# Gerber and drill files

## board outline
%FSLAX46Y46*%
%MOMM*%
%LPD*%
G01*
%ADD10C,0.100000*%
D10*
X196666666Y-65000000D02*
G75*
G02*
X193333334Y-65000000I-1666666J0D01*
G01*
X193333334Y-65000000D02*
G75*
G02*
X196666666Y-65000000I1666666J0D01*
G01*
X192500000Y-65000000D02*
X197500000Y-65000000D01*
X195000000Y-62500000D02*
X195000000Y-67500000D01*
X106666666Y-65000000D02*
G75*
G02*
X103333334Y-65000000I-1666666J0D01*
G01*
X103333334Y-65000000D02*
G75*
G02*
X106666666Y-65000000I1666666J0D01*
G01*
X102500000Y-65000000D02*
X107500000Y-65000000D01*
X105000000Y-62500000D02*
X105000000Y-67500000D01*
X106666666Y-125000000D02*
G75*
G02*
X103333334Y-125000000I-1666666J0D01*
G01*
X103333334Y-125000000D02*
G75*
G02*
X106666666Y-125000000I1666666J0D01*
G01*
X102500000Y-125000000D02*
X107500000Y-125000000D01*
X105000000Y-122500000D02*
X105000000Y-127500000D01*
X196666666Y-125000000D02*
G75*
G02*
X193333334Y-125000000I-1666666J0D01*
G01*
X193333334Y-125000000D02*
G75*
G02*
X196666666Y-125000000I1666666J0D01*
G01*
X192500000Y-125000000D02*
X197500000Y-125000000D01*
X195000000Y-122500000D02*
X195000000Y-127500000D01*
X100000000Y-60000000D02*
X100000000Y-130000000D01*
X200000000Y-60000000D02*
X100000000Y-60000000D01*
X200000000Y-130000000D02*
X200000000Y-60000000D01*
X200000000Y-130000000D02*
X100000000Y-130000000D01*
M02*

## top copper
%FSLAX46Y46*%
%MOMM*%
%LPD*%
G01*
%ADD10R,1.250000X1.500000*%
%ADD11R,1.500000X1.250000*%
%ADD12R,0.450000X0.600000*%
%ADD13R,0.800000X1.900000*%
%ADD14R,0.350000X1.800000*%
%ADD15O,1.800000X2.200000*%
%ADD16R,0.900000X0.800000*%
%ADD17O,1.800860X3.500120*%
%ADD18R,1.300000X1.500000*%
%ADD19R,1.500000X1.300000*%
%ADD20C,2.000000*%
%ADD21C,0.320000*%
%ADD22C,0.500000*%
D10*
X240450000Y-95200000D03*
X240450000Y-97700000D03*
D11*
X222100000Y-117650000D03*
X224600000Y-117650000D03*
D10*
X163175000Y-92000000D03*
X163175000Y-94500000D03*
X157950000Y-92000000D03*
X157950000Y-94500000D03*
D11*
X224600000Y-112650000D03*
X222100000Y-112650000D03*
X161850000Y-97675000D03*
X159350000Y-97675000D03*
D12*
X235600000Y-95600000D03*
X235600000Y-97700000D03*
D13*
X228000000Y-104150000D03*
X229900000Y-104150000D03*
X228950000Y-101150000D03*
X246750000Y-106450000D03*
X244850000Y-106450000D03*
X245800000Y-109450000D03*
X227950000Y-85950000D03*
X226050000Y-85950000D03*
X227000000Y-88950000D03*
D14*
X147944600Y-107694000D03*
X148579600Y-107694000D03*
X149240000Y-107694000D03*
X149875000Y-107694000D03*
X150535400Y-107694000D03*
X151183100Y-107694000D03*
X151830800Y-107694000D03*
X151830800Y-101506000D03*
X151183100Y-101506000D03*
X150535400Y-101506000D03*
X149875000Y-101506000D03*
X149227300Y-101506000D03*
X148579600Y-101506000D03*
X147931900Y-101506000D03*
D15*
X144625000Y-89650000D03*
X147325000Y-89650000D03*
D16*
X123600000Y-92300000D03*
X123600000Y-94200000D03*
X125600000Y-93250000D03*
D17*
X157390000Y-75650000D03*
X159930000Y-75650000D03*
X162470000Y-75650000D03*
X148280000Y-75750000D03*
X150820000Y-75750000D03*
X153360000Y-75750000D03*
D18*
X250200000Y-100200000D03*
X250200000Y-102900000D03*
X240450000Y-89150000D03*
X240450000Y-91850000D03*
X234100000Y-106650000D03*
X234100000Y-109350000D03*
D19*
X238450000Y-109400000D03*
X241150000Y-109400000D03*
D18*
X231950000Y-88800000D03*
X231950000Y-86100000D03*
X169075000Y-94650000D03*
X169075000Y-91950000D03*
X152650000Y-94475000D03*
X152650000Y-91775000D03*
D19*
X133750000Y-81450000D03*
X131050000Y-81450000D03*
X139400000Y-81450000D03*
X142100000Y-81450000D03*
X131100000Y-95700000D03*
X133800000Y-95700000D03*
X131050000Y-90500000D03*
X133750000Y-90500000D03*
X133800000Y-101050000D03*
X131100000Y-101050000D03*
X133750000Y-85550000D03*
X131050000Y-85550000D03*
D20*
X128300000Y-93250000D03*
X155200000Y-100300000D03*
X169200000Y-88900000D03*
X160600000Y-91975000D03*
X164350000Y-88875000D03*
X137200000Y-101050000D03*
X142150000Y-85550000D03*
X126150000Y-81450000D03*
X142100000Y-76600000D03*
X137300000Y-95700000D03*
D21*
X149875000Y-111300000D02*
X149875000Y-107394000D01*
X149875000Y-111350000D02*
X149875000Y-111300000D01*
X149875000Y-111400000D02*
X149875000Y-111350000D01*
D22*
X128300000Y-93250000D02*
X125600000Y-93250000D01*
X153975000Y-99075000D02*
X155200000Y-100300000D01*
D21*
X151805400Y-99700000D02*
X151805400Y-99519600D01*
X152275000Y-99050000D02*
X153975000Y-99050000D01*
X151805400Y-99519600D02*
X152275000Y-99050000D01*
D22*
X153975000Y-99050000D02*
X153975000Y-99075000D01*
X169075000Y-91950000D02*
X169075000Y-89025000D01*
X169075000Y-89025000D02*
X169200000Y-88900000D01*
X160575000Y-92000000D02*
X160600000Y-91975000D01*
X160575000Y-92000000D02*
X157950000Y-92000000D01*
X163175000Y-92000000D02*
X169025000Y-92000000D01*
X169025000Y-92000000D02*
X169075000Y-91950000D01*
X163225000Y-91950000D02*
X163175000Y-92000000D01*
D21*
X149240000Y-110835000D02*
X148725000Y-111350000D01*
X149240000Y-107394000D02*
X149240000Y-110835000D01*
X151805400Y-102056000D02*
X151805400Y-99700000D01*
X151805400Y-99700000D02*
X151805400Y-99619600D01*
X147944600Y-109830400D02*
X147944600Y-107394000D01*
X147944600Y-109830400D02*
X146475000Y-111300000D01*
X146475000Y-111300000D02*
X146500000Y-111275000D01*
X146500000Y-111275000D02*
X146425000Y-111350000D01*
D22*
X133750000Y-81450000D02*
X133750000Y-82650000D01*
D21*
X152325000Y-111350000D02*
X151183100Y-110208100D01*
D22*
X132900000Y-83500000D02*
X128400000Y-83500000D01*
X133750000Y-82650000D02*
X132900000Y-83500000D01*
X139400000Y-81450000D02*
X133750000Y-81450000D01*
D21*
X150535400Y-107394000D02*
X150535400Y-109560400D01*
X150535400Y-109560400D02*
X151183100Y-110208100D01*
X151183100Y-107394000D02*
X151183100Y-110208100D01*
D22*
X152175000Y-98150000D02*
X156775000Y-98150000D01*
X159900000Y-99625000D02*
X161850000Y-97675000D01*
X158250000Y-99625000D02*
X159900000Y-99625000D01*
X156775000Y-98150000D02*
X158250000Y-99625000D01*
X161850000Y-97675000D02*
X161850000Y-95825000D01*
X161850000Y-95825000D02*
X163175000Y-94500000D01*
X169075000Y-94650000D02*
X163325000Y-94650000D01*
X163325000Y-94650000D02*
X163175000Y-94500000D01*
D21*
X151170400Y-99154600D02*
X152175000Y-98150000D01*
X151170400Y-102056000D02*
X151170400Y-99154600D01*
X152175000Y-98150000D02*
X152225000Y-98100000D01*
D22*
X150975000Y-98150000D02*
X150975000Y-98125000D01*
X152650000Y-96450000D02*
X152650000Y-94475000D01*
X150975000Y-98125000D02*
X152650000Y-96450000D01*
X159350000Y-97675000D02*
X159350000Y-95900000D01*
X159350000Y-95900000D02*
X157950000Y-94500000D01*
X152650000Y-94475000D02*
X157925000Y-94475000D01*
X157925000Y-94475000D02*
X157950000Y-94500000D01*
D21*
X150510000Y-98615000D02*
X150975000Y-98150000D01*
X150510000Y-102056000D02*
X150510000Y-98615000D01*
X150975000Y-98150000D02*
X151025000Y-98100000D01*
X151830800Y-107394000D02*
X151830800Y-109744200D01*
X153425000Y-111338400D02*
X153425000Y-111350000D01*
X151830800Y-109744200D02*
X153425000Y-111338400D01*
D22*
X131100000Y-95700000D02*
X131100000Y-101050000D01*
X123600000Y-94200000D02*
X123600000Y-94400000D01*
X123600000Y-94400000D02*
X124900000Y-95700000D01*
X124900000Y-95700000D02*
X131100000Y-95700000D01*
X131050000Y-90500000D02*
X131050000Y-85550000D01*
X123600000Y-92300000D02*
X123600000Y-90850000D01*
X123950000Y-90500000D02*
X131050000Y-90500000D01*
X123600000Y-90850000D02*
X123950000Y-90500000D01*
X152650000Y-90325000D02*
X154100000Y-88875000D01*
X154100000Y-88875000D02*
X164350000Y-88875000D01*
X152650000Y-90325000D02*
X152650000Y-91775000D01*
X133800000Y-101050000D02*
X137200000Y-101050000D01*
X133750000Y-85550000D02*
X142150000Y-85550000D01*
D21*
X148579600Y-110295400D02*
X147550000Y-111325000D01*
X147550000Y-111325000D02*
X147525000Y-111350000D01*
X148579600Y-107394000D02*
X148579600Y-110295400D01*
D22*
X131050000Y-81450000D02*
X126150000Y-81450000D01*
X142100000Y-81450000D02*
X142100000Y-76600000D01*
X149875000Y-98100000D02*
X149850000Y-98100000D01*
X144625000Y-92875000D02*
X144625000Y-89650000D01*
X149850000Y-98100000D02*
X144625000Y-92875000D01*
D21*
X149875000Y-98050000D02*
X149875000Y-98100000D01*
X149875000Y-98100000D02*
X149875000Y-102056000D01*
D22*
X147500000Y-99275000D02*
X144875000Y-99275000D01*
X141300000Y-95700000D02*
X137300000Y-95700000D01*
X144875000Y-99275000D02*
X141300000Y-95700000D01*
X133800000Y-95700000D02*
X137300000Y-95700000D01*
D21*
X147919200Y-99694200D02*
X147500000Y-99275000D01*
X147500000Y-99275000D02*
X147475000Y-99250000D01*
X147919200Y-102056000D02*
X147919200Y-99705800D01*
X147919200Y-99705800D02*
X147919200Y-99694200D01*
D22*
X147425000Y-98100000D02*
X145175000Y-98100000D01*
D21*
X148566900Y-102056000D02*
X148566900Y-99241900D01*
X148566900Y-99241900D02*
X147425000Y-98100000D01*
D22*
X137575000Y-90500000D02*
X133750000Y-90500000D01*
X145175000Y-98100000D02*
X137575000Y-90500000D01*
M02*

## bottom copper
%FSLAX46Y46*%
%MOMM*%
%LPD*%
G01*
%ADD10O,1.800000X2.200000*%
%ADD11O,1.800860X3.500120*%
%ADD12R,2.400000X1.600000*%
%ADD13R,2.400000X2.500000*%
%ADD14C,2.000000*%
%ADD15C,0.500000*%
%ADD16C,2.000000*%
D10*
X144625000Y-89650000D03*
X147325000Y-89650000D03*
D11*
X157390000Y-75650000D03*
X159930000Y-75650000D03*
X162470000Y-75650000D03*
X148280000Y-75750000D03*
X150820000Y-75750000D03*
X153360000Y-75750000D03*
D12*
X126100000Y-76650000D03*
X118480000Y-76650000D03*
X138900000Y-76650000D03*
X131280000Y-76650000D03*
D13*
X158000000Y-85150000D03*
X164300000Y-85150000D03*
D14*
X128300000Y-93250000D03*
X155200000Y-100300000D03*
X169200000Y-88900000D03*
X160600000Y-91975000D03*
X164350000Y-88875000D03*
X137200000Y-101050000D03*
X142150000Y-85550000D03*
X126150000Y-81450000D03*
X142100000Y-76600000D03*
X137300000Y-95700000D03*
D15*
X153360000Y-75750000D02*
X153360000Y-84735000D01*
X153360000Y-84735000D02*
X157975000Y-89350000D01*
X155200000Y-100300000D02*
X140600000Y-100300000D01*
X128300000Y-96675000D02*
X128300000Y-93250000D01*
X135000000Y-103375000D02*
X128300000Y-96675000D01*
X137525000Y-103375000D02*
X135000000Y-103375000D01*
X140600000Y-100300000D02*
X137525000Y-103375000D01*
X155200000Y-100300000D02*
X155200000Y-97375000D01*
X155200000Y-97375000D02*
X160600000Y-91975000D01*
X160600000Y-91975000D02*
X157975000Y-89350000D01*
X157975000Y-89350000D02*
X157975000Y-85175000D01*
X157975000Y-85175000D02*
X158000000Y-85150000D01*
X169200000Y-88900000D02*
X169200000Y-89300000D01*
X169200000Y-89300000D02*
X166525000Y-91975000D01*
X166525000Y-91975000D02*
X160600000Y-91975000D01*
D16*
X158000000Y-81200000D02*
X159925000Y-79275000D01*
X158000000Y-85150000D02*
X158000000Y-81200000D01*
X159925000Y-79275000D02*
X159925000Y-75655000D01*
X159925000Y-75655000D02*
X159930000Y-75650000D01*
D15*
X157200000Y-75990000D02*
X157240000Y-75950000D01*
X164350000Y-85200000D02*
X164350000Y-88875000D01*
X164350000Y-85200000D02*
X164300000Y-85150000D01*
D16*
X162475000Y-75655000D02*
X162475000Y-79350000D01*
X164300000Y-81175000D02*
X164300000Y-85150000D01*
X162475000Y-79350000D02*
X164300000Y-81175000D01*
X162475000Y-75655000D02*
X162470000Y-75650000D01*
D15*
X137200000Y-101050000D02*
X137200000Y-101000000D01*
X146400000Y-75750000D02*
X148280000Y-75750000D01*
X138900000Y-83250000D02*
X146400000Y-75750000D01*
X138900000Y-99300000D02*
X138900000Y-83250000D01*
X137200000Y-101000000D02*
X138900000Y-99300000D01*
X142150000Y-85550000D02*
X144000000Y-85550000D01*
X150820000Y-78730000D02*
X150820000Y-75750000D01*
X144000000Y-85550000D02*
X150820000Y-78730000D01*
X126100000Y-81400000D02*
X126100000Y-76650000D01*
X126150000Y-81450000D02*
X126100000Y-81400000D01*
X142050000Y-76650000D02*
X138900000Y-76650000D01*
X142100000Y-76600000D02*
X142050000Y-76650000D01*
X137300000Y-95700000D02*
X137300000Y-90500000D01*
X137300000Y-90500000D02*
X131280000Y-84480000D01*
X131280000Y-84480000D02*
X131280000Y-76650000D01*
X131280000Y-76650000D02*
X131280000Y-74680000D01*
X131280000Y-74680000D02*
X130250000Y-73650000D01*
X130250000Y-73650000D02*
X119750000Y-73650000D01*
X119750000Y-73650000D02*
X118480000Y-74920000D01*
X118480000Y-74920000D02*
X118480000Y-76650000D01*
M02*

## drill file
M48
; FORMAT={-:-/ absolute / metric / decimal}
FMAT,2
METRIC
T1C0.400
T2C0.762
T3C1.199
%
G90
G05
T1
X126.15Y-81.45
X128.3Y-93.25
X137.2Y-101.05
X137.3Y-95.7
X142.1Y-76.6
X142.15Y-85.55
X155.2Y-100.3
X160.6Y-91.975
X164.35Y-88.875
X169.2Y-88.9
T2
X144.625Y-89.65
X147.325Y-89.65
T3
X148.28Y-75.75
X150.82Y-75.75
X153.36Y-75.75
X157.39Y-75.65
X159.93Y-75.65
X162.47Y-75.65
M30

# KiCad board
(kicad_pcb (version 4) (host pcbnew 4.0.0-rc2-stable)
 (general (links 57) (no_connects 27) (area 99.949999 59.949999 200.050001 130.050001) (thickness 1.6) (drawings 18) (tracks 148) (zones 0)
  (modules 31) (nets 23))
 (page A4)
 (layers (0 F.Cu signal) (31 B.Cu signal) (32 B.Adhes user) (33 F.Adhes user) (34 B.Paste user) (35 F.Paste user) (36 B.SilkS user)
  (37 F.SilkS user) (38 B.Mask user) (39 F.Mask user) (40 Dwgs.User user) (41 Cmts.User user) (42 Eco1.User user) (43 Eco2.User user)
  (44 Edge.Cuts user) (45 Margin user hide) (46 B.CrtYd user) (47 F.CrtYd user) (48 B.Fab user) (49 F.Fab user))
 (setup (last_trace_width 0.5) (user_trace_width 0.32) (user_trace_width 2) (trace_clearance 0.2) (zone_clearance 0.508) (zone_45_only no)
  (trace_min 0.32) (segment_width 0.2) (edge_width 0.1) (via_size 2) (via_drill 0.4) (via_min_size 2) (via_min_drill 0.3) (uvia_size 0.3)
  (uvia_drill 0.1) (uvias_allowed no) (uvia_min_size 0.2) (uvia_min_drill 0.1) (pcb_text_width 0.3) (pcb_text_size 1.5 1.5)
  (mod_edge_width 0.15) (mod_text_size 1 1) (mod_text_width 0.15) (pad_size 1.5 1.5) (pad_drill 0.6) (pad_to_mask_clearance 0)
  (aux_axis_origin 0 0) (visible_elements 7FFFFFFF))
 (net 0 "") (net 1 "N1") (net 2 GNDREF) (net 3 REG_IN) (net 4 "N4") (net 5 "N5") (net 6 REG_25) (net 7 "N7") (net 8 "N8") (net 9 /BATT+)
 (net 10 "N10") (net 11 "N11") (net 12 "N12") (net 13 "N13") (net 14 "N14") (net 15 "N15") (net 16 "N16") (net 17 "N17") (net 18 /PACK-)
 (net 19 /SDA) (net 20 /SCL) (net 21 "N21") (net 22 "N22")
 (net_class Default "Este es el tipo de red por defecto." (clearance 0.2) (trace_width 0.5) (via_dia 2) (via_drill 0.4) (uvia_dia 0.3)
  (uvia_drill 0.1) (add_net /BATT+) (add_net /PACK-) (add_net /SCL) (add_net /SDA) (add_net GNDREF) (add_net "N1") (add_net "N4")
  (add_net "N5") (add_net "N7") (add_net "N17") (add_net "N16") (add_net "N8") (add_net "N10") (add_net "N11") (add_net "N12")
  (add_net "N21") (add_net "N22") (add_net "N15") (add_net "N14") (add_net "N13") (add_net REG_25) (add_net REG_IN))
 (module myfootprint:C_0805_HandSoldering (layer F.Cu) (at 240.45 96.45 270)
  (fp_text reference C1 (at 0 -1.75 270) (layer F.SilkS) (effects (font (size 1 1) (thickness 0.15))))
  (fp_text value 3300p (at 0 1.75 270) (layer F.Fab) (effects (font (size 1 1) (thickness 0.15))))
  (pad 1 smd rect (at -1.25 0 270) (size 1.5 1.25) (layers F.Cu F.Paste F.Mask) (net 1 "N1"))
  (pad 2 smd rect (at 1.25 0 270) (size 1.5 1.25) (layers F.Cu F.Paste F.Mask) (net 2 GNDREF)))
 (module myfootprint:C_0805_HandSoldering (layer F.Cu) (at 223.35 117.65)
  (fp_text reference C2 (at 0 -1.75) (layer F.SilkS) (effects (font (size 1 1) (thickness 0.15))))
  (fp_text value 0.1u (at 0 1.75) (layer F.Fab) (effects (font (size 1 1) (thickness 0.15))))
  (pad 1 smd rect (at -1.25 0) (size 1.5 1.25) (layers F.Cu F.Paste F.Mask) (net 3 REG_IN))
  (pad 2 smd rect (at 1.25 0) (size 1.5 1.25) (layers F.Cu F.Paste F.Mask) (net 2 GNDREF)))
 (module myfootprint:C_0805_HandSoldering (layer F.Cu) (at 163.175 93.25 270)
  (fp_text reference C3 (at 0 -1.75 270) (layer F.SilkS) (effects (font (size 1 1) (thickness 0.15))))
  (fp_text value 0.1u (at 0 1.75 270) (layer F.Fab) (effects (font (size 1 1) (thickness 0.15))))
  (pad 1 smd rect (at -1.25 0 270) (size 1.5 1.25) (layers F.Cu F.Paste F.Mask) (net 2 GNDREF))
  (pad 2 smd rect (at 1.25 0 270) (size 1.5 1.25) (layers F.Cu F.Paste F.Mask) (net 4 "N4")))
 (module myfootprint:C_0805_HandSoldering (layer F.Cu) (at 157.95 93.25 270)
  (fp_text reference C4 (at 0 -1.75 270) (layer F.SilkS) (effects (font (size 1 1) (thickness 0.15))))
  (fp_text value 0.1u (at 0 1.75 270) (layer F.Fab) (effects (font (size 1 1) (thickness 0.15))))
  (pad 1 smd rect (at -1.25 0 270) (size 1.5 1.25) (layers F.Cu F.Paste F.Mask) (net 2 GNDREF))
  (pad 2 smd rect (at 1.25 0 270) (size 1.5 1.25) (layers F.Cu F.Paste F.Mask) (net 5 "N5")))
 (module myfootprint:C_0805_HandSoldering (layer F.Cu) (at 223.35 112.65 180)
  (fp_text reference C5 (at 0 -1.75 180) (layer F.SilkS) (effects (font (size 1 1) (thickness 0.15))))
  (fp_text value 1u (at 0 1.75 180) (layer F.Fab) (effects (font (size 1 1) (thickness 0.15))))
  (pad 1 smd rect (at -1.25 0 180) (size 1.5 1.25) (layers F.Cu F.Paste F.Mask) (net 2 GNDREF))
  (pad 2 smd rect (at 1.25 0 180) (size 1.5 1.25) (layers F.Cu F.Paste F.Mask) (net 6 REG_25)))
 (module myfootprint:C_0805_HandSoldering (layer F.Cu) (at 160.6 97.675 180)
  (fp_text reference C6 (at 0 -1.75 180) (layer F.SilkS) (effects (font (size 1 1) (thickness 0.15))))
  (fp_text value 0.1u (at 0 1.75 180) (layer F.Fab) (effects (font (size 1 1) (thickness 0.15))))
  (pad 1 smd rect (at -1.25 0 180) (size 1.5 1.25) (layers F.Cu F.Paste F.Mask) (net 4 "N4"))
  (pad 2 smd rect (at 1.25 0 180) (size 1.5 1.25) (layers F.Cu F.Paste F.Mask) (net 5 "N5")))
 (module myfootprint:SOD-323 (layer F.Cu) (at 235.6 96.65 270)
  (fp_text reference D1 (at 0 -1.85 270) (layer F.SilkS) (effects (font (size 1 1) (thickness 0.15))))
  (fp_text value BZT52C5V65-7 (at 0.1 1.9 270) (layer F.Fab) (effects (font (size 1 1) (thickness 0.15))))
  (pad 1 smd rect (at -1.05 0 270) (size 0.6 0.45) (layers F.Cu F.Paste F.Mask) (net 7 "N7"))
  (pad 2 smd rect (at 1.05 0 270) (size 0.6 0.45) (layers F.Cu F.Paste F.Mask) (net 2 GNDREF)))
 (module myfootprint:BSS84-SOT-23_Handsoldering (layer F.Cu) (at 228.95 102.65 90)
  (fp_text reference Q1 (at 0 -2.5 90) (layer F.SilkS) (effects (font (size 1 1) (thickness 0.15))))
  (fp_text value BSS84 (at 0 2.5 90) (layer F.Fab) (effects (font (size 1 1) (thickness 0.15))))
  (pad 1 smd rect (at -1.5 -0.95 90) (size 1.9 0.8) (layers F.Cu F.Paste F.Mask) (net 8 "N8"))
  (pad 2 smd rect (at -1.5 0.95 90) (size 1.9 0.8) (layers F.Cu F.Paste F.Mask) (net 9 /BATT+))
  (pad 3 smd rect (at 1.5 0 90) (size 1.9 0.8) (layers F.Cu F.Paste F.Mask) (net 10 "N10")))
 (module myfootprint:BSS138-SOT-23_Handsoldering (layer F.Cu) (at 245.8 107.95 270)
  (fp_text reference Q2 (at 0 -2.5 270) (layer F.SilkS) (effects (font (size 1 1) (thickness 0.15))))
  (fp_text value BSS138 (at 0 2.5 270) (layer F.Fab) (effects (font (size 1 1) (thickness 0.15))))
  (pad 1 smd rect (at -1.5 -0.95 270) (size 1.9 0.8) (layers F.Cu F.Paste F.Mask) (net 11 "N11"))
  (pad 2 smd rect (at -1.5 0.95 270) (size 1.9 0.8) (layers F.Cu F.Paste F.Mask) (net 2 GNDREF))
  (pad 3 smd rect (at 1.5 0 270) (size 1.9 0.8) (layers F.Cu F.Paste F.Mask) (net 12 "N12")))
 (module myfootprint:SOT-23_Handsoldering (layer F.Cu) (at 227 87.45 270)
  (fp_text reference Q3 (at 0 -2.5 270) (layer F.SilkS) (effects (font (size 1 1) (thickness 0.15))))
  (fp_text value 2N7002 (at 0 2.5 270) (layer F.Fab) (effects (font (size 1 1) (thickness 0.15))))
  (pad 1 smd rect (at -1.5 -0.95 270) (size 1.9 0.8) (layers F.Cu F.Paste F.Mask) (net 7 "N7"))
  (pad 2 smd rect (at -1.5 0.95 270) (size 1.9 0.8) (layers F.Cu F.Paste F.Mask) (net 3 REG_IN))
  (pad 3 smd rect (at 1.5 0 270) (size 1.9 0.8) (layers F.Cu F.Paste F.Mask) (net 9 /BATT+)))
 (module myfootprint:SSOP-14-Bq (layer F.Cu) (at 149.875 104.6)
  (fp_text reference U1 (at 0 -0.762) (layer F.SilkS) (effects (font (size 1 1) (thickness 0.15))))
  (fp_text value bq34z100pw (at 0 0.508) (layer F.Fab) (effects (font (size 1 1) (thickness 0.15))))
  (pad 1 smd rect (at -1.9304 2.794) (size 0.35 1.8) (drill (offset 0 0.3)) (layers F.Cu F.Paste F.Mask) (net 2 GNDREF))
  (pad 2 smd rect (at -1.2954 2.794) (size 0.35 1.8) (drill (offset 0 0.3)) (layers F.Cu F.Paste F.Mask) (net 11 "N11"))
  (pad 3 smd rect (at -0.635 2.794) (size 0.35 1.8) (drill (offset 0 0.3)) (layers F.Cu F.Paste F.Mask) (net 2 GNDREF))
  (pad 4 smd rect (at 0 2.794) (size 0.35 1.8) (drill (offset 0 0.3)) (layers F.Cu F.Paste F.Mask) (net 1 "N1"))
  (pad 5 smd rect (at 0.6604 2.794) (size 0.35 1.8) (drill (offset 0 0.3)) (layers F.Cu F.Paste F.Mask) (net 3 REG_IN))
  (pad 6 smd rect (at 1.3081 2.794) (size 0.35 1.8) (drill (offset 0 0.3)) (layers F.Cu F.Paste F.Mask) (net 3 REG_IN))
  (pad 7 smd rect (at 1.9558 2.794) (size 0.35 1.8) (drill (offset 0 0.3)) (layers F.Cu F.Paste F.Mask) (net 6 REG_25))
  (pad 8 smd rect (at 1.9558 -2.794) (size 0.35 1.8) (drill (offset 0 -0.3)) (layers F.Cu F.Paste F.Mask) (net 2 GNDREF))
  (pad 9 smd rect (at 1.3081 -2.794) (size 0.35 1.8) (drill (offset 0 -0.3)) (layers F.Cu F.Paste F.Mask) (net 4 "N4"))
  (pad 10 smd rect (at 0.6604 -2.794) (size 0.35 1.8) (drill (offset 0 -0.3)) (layers F.Cu F.Paste F.Mask) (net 5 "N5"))
  (pad 11 smd rect (at 0 -2.794) (size 0.35 1.8) (drill (offset 0 -0.3)) (layers F.Cu F.Paste F.Mask) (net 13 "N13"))
  (pad 12 smd rect (at -0.6477 -2.794) (size 0.35 1.8) (drill (offset 0 -0.3)) (layers F.Cu F.Paste F.Mask))
  (pad 13 smd rect (at -1.2954 -2.794) (size 0.35 1.8) (drill (offset 0 -0.3)) (layers F.Cu F.Paste F.Mask) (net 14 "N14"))
  (pad 14 smd rect (at -1.9431 -2.794) (size 0.35 1.8) (drill (offset 0 -0.3)) (layers F.Cu F.Paste F.Mask) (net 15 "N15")))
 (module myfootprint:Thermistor (layer F.Cu) (at 147.325 89.65 180)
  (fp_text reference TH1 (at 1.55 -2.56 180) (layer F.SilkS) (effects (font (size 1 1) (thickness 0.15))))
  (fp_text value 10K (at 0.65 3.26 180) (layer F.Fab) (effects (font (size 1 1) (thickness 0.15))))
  (pad 2 thru_hole oval (at 2.7 0 180) (size 1.8 2.2) (drill 0.762) (layers *.Cu *.Mask F.SilkS) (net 13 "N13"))
  (pad 1 thru_hole oval (at 0 0 180) (size 1.8 2.2) (drill 0.762) (layers *.Cu *.Mask F.SilkS) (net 6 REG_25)))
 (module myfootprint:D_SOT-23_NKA (layer F.Cu) (at 124.6 93.25)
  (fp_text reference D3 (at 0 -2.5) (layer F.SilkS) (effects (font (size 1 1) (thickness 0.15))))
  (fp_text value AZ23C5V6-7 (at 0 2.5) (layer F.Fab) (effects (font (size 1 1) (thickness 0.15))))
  (pad 2 smd rect (at -1 -0.95) (size 0.9 0.8) (layers F.Cu F.Paste F.Mask) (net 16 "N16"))
  (pad 1 smd rect (at -1 0.95) (size 0.9 0.8) (layers F.Cu F.Paste F.Mask) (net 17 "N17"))
  (pad 3 smd rect (at 1 0) (size 0.9 0.8) (layers F.Cu F.Paste F.Mask) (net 2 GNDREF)))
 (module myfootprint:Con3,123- (layer F.Cu) (at 161.2 75.65)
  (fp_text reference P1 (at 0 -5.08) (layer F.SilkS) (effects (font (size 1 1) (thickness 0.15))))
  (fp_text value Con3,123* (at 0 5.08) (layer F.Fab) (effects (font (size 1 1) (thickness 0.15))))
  (pad 1 thru_hole oval (at -3.81 0) (size 1.80086 3.50012) (drill 1.19888) (layers *.Cu *.Mask) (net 9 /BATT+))
  (pad 2 thru_hole oval (at -1.27 0) (size 1.80086 3.50012) (drill 1.19888) (layers *.Cu *.Mask) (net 2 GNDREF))
  (pad 3 thru_hole oval (at 1.27 0) (size 1.80086 3.50012) (drill 1.19888) (layers *.Cu *.Mask) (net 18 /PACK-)))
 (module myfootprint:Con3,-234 (layer F.Cu) (at 149.55 75.75)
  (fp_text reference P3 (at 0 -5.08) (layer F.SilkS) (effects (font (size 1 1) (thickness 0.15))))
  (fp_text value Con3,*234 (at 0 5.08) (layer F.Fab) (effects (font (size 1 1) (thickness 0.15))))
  (pad 2 thru_hole oval (at -1.27 0) (size 1.80086 3.50012) (drill 1.19888) (layers *.Cu *.Mask) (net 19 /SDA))
  (pad 3 thru_hole oval (at 1.27 0) (size 1.80086 3.50012) (drill 1.19888) (layers *.Cu *.Mask) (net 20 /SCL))
  (pad 4 thru_hole oval (at 3.81 0) (size 1.80086 3.50012) (drill 1.19888) (layers *.Cu *.Mask) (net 2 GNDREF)))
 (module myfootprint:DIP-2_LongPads (layer B.Cu) (at 126.1 76.65 180)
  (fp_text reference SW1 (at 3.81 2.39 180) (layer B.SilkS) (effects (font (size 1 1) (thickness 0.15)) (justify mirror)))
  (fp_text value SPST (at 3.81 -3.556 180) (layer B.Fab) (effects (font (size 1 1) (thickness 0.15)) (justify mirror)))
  (pad 1 smd rect (at 0 0 180) (size 2.4 1.6) (layers B.Cu B.Paste B.Mask) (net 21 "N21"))
  (pad 2 smd rect (at 7.62 0 180) (size 2.4 1.6) (layers B.Cu B.Paste B.Mask) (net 15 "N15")))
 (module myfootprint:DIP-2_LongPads (layer B.Cu) (at 138.9 76.65 180)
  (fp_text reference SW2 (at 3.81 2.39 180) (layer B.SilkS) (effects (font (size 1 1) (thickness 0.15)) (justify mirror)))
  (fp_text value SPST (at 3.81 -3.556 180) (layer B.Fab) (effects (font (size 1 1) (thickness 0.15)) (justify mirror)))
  (pad 1 smd rect (at 0 0 180) (size 2.4 1.6) (layers B.Cu B.Paste B.Mask) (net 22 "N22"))
  (pad 2 smd rect (at 7.62 0 180) (size 2.4 1.6) (layers B.Cu B.Paste B.Mask) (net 15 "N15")))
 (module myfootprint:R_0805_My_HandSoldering (layer F.Cu) (at 250.2 101.55 270)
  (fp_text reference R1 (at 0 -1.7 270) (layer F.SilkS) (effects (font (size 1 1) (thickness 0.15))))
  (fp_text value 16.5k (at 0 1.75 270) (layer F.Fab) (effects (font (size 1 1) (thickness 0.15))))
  (pad 1 smd rect (at -1.35 0 270) (size 1.5 1.3) (layers F.Cu F.Paste F.Mask) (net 1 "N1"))
  (pad 2 smd rect (at 1.35 0 270) (size 1.5 1.3) (layers F.Cu F.Paste F.Mask) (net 2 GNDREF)))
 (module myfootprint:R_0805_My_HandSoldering (layer F.Cu) (at 240.45 90.5 270)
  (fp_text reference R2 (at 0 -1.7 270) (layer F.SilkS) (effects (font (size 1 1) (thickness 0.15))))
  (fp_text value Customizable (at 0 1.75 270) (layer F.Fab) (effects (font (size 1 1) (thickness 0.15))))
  (pad 1 smd rect (at -1.35 0 270) (size 1.5 1.3) (layers F.Cu F.Paste F.Mask) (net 10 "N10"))
  (pad 2 smd rect (at 1.35 0 270) (size 1.5 1.3) (layers F.Cu F.Paste F.Mask) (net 1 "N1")))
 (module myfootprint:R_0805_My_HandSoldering (layer F.Cu) (at 234.1 108 270)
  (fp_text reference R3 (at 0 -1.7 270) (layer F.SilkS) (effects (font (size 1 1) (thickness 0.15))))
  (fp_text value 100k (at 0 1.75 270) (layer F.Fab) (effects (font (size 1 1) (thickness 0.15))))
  (pad 1 smd rect (at -1.35 0 270) (size 1.5 1.3) (layers F.Cu F.Paste F.Mask) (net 9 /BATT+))
  (pad 2 smd rect (at 1.35 0 270) (size 1.5 1.3) (layers F.Cu F.Paste F.Mask) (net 8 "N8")))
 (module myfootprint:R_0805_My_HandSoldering (layer F.Cu) (at 239.8 109.4)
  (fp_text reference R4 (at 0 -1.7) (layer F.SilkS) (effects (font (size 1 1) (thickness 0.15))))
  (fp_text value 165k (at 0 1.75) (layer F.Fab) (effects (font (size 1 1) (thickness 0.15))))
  (pad 1 smd rect (at -1.35 0) (size 1.5 1.3) (layers F.Cu F.Paste F.Mask) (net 8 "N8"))
  (pad 2 smd rect (at 1.35 0) (size 1.5 1.3) (layers F.Cu F.Paste F.Mask) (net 12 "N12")))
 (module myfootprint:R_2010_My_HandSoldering (layer B.Cu) (at 161.15 85.15)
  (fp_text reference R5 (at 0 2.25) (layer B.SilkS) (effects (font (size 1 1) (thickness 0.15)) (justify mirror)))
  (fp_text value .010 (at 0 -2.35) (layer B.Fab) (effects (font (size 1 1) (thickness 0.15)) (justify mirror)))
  (pad 1 smd rect (at -3.15 0) (size 2.4 2.5) (layers B.Cu B.Paste B.Mask) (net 2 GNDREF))
  (pad 2 smd rect (at 3.15 0) (size 2.4 2.5) (layers B.Cu B.Paste B.Mask) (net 18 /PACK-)))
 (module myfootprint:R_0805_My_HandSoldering (layer F.Cu) (at 231.95 87.45 90)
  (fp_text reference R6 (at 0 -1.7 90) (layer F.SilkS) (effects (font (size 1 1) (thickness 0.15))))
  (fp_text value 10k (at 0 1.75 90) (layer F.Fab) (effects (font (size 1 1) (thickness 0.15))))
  (pad 1 smd rect (at -1.35 0 90) (size 1.5 1.3) (layers F.Cu F.Paste F.Mask) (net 9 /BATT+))
  (pad 2 smd rect (at 1.35 0 90) (size 1.5 1.3) (layers F.Cu F.Paste F.Mask) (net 7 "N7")))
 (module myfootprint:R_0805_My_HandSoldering (layer F.Cu) (at 169.075 93.3 90)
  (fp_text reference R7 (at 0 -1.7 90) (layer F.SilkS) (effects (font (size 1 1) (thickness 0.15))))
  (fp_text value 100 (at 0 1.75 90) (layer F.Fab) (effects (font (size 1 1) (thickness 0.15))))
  (pad 1 smd rect (at -1.35 0 90) (size 1.5 1.3) (layers F.Cu F.Paste F.Mask) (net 4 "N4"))
  (pad 2 smd rect (at 1.35 0 90) (size 1.5 1.3) (layers F.Cu F.Paste F.Mask) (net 2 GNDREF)))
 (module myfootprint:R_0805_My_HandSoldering (layer F.Cu) (at 152.65 93.125 90)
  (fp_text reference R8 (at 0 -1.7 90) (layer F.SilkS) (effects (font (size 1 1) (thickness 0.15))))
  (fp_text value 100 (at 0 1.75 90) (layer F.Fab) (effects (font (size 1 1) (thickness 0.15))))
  (pad 1 smd rect (at -1.35 0 90) (size 1.5 1.3) (layers F.Cu F.Paste F.Mask) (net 5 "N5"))
  (pad 2 smd rect (at 1.35 0 90) (size 1.5 1.3) (layers F.Cu F.Paste F.Mask) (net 18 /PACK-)))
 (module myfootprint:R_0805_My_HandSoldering (layer F.Cu) (at 132.4 81.45 180)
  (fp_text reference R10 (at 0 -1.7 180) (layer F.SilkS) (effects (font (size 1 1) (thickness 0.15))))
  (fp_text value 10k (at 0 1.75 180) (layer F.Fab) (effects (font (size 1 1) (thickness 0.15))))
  (pad 1 smd rect (at -1.35 0 180) (size 1.5 1.3) (layers F.Cu F.Paste F.Mask) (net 3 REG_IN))
  (pad 2 smd rect (at 1.35 0 180) (size 1.5 1.3) (layers F.Cu F.Paste F.Mask) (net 21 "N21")))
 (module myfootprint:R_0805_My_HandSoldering (layer F.Cu) (at 140.75 81.45)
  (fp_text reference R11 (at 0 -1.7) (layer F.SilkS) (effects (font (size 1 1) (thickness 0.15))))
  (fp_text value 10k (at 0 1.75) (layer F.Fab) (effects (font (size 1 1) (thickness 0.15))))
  (pad 1 smd rect (at -1.35 0) (size 1.5 1.3) (layers F.Cu F.Paste F.Mask) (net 3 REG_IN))
  (pad 2 smd rect (at 1.35 0) (size 1.5 1.3) (layers F.Cu F.Paste F.Mask) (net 22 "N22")))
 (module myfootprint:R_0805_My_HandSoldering (layer F.Cu) (at 132.45 95.7)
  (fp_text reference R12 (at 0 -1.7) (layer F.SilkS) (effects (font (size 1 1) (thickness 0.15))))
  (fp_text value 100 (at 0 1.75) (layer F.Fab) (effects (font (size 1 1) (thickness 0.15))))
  (pad 1 smd rect (at -1.35 0) (size 1.5 1.3) (layers F.Cu F.Paste F.Mask) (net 17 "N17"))
  (pad 2 smd rect (at 1.35 0) (size 1.5 1.3) (layers F.Cu F.Paste F.Mask) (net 15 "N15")))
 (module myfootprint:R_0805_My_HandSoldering (layer F.Cu) (at 132.4 90.5)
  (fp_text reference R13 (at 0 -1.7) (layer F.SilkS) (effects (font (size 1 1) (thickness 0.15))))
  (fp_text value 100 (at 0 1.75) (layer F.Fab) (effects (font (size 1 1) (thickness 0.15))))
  (pad 1 smd rect (at -1.35 0) (size 1.5 1.3) (layers F.Cu F.Paste F.Mask) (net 16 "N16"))
  (pad 2 smd rect (at 1.35 0) (size 1.5 1.3) (layers F.Cu F.Paste F.Mask) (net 14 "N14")))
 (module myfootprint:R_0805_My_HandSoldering (layer F.Cu) (at 132.45 101.05 180)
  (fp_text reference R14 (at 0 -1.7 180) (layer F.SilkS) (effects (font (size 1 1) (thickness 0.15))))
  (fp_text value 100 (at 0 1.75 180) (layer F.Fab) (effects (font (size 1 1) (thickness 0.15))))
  (pad 1 smd rect (at -1.35 0 180) (size 1.5 1.3) (layers F.Cu F.Paste F.Mask) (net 19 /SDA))
  (pad 2 smd rect (at 1.35 0 180) (size 1.5 1.3) (layers F.Cu F.Paste F.Mask) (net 17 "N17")))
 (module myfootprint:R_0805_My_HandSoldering (layer F.Cu) (at 132.4 85.55 180)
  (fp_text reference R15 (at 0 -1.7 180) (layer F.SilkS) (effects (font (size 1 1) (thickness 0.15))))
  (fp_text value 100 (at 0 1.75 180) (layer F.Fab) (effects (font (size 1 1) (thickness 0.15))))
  (pad 1 smd rect (at -1.35 0 180) (size 1.5 1.3) (layers F.Cu F.Paste F.Mask) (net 20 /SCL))
  (pad 2 smd rect (at 1.35 0 180) (size 1.5 1.3) (layers F.Cu F.Paste F.Mask) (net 16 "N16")))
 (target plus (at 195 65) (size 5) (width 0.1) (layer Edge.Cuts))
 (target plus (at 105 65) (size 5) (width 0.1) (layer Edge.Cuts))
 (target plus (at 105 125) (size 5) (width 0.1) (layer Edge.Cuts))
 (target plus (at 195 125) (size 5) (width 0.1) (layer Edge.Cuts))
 (gr_line (start 100 60) (end 100 130) (angle 90) (layer Edge.Cuts) (width 0.1))
 (gr_line (start 200 60) (end 100 60) (angle 90) (layer Edge.Cuts) (width 0.1))
 (gr_line (start 200 130) (end 200 60) (angle 90) (layer Edge.Cuts) (width 0.1))
 (gr_line (start 200 130) (end 100 130) (angle 90) (layer Edge.Cuts) (width 0.1))
 (segment (start 149.875 111.3) (end 149.875 107.394) (width 0.32) (layer F.Cu) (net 1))
 (segment (start 149.875 111.35) (end 149.875 111.3) (width 0.32) (layer F.Cu) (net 1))
 (segment (start 149.875 111.4) (end 149.875 111.35) (width 0.32) (layer F.Cu) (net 1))
 (segment (start 153.36 75.75) (end 153.36 84.735) (width 0.5) (layer B.Cu) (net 2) (status 400000))
 (segment (start 153.36 84.735) (end 157.975 89.35) (width 0.5) (layer B.Cu) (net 2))
 (segment (start 155.2 100.3) (end 140.6 100.3) (width 0.5) (layer B.Cu) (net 2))
 (via (at 128.3 93.25) (size 2) (drill 0.4) (layers F.Cu B.Cu) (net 2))
 (segment (start 128.3 93.25) (end 125.6 93.25) (width 0.5) (layer F.Cu) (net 2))
 (segment (start 128.3 96.675) (end 128.3 93.25) (width 0.5) (layer B.Cu) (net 2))
 (segment (start 135 103.375) (end 128.3 96.675) (width 0.5) (layer B.Cu) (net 2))
 (segment (start 137.525 103.375) (end 135 103.375) (width 0.5) (layer B.Cu) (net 2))
 (segment (start 140.6 100.3) (end 137.525 103.375) (width 0.5) (layer B.Cu) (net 2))
 (segment (start 155.2 100.3) (end 155.2 97.375) (width 0.5) (layer B.Cu) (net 2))
 (segment (start 153.975 99.075) (end 155.2 100.3) (width 0.5) (layer F.Cu) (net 2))
 (via (at 155.2 100.3) (size 2) (drill 0.4) (layers F.Cu B.Cu) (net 2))
 (segment (start 151.8054 99.7) (end 151.8054 99.5196) (width 0.32) (layer F.Cu) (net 2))
 (segment (start 152.275 99.05) (end 153.975 99.05) (width 0.32) (layer F.Cu) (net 2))
 (segment (start 151.8054 99.5196) (end 152.275 99.05) (width 0.32) (layer F.Cu) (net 2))
 (segment (start 153.975 99.05) (end 153.975 99.075) (width 0.5) (layer F.Cu) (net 2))
 (segment (start 155.2 97.375) (end 160.6 91.975) (width 0.5) (layer B.Cu) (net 2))
 (segment (start 160.6 91.975) (end 157.975 89.35) (width 0.5) (layer B.Cu) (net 2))
 (segment (start 157.975 89.35) (end 157.975 85.175) (width 0.5) (layer B.Cu) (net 2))
 (segment (start 157.975 85.175) (end 158 85.15) (width 0.5) (layer B.Cu) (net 2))
 (segment (start 169.2 88.9) (end 169.2 89.3) (width 0.5) (layer B.Cu) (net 2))
 (segment (start 169.2 89.3) (end 166.525 91.975) (width 0.5) (layer B.Cu) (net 2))
 (segment (start 166.525 91.975) (end 160.6 91.975) (width 0.5) (layer B.Cu) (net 2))
 (segment (start 169.075 91.95) (end 169.075 89.025) (width 0.5) (layer F.Cu) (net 2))
 (via (at 169.2 88.9) (size 2) (drill 0.4) (layers F.Cu B.Cu) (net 2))
 (segment (start 169.075 89.025) (end 169.2 88.9) (width 0.5) (layer F.Cu) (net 2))
 (segment (start 160.575 92) (end 160.6 91.975) (width 0.5) (layer F.Cu) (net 2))
 (segment (start 160.575 92) (end 157.95 92) (width 0.5) (layer F.Cu) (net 2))
 (via (at 160.6 91.975) (size 2) (drill 0.4) (layers F.Cu B.Cu) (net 2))
 (segment (start 163.175 92) (end 169.025 92) (width 0.5) (layer F.Cu) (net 2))
 (segment (start 169.025 92) (end 169.075 91.95) (width 0.5) (layer F.Cu) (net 2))
 (segment (start 163.225 91.95) (end 163.175 92) (width 0.5) (layer F.Cu) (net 2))
 (segment (start 158 81.2) (end 159.925 79.275) (width 2) (layer B.Cu) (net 2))
 (segment (start 158 85.15) (end 158 81.2) (width 2) (layer B.Cu) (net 2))
 (segment (start 159.925 79.275) (end 159.925 75.655) (width 2) (layer B.Cu) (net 2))
 (segment (start 159.925 75.655) (end 159.93 75.65) (width 2) (layer B.Cu) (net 2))
 (segment (start 149.24 110.835) (end 148.725 111.35) (width 0.32) (layer F.Cu) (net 2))
 (segment (start 149.24 107.394) (end 149.24 110.835) (width 0.32) (layer F.Cu) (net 2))
 (segment (start 151.8054 102.056) (end 151.8054 99.7) (width 0.32) (layer F.Cu) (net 2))
 (segment (start 151.8054 99.7) (end 151.8054 99.6196) (width 0.32) (layer F.Cu) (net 2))
 (segment (start 147.9446 109.8304) (end 147.9446 107.394) (width 0.32) (layer F.Cu) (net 2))
 (segment (start 147.9446 109.8304) (end 146.475 111.3) (width 0.32) (layer F.Cu) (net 2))
 (segment (start 146.475 111.3) (end 146.5 111.275) (width 0.32) (layer F.Cu) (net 2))
 (segment (start 146.5 111.275) (end 146.425 111.35) (width 0.32) (layer F.Cu) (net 2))
 (segment (start 133.75 81.45) (end 133.75 82.65) (width 0.5) (layer F.Cu) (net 3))
 (segment (start 152.325 111.35) (end 151.1831 110.2081) (width 0.32) (layer F.Cu) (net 3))
 (segment (start 132.9 83.5) (end 128.4 83.5) (width 0.5) (layer F.Cu) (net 3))
 (segment (start 133.75 82.65) (end 132.9 83.5) (width 0.5) (layer F.Cu) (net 3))
 (segment (start 139.4 81.45) (end 133.75 81.45) (width 0.5) (layer F.Cu) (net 3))
 (segment (start 150.5354 107.394) (end 150.5354 109.5604) (width 0.32) (layer F.Cu) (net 3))
 (segment (start 150.5354 109.5604) (end 151.1831 110.2081) (width 0.32) (layer F.Cu) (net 3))
 (segment (start 151.1831 107.394) (end 151.1831 110.2081) (width 0.32) (layer F.Cu) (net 3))
 (segment (start 152.175 98.15) (end 156.775 98.15) (width 0.5) (layer F.Cu) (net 4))
 (segment (start 159.9 99.625) (end 161.85 97.675) (width 0.5) (layer F.Cu) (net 4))
 (segment (start 158.25 99.625) (end 159.9 99.625) (width 0.5) (layer F.Cu) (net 4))
 (segment (start 156.775 98.15) (end 158.25 99.625) (width 0.5) (layer F.Cu) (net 4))
 (segment (start 161.85 97.675) (end 161.85 95.825) (width 0.5) (layer F.Cu) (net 4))
 (segment (start 161.85 95.825) (end 163.175 94.5) (width 0.5) (layer F.Cu) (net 4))
 (segment (start 169.075 94.65) (end 163.325 94.65) (width 0.5) (layer F.Cu) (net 4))
 (segment (start 163.325 94.65) (end 163.175 94.5) (width 0.5) (layer F.Cu) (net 4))
 (segment (start 151.1704 99.1546) (end 152.175 98.15) (width 0.32) (layer F.Cu) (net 4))
 (segment (start 151.1704 102.056) (end 151.1704 99.1546) (width 0.32) (layer F.Cu) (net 4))
 (segment (start 152.175 98.15) (end 152.225 98.1) (width 0.32) (layer F.Cu) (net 4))
 (segment (start 150.975 98.15) (end 150.975 98.125) (width 0.5) (layer F.Cu) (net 5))
 (segment (start 152.65 96.45) (end 152.65 94.475) (width 0.5) (layer F.Cu) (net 5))
 (segment (start 150.975 98.125) (end 152.65 96.45) (width 0.5) (layer F.Cu) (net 5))
 (segment (start 159.35 97.675) (end 159.35 95.9) (width 0.5) (layer F.Cu) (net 5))
 (segment (start 159.35 95.9) (end 157.95 94.5) (width 0.5) (layer F.Cu) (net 5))
 (segment (start 152.65 94.475) (end 157.925 94.475) (width 0.5) (layer F.Cu) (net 5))
 (segment (start 157.925 94.475) (end 157.95 94.5) (width 0.5) (layer F.Cu) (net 5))
 (segment (start 150.51 98.615) (end 150.975 98.15) (width 0.32) (layer F.Cu) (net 5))
 (segment (start 150.51 102.056) (end 150.51 98.615) (width 0.32) (layer F.Cu) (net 5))
 (segment (start 150.975 98.15) (end 151.025 98.1) (width 0.32) (layer F.Cu) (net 5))
 (segment (start 151.8308 107.394) (end 151.8308 109.7442) (width 0.32) (layer F.Cu) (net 6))
 (segment (start 153.425 111.3384) (end 153.425 111.35) (width 0.32) (layer F.Cu) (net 6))
 (segment (start 151.8308 109.7442) (end 153.425 111.3384) (width 0.32) (layer F.Cu) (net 6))
 (segment (start 131.1 95.7) (end 131.1 101.05) (width 0.5) (layer F.Cu) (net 17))
 (segment (start 123.6 94.2) (end 123.6 94.4) (width 0.5) (layer F.Cu) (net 17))
 (segment (start 123.6 94.4) (end 124.9 95.7) (width 0.5) (layer F.Cu) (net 17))
 (segment (start 124.9 95.7) (end 131.1 95.7) (width 0.5) (layer F.Cu) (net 17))
 (segment (start 131.05 90.5) (end 131.05 85.55) (width 0.5) (layer F.Cu) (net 16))
 (segment (start 123.6 92.3) (end 123.6 90.85) (width 0.5) (layer F.Cu) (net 16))
 (segment (start 123.95 90.5) (end 131.05 90.5) (width 0.5) (layer F.Cu) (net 16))
 (segment (start 123.6 90.85) (end 123.95 90.5) (width 0.5) (layer F.Cu) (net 16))
 (segment (start 157.2 75.99) (end 157.24 75.95) (width 0.5) (layer B.Cu) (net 9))
 (segment (start 164.35 85.2) (end 164.35 88.875) (width 0.5) (layer B.Cu) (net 18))
 (segment (start 152.65 90.325) (end 154.1 88.875) (width 0.5) (layer F.Cu) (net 18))
 (segment (start 154.1 88.875) (end 164.35 88.875) (width 0.5) (layer F.Cu) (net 18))
 (via (at 164.35 88.875) (size 2) (drill 0.4) (layers F.Cu B.Cu) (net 18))
 (segment (start 152.65 90.325) (end 152.65 91.775) (width 0.5) (layer F.Cu) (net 18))
 (segment (start 164.35 85.2) (end 164.3 85.15) (width 0.5) (layer B.Cu) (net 18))
 (segment (start 162.475 75.655) (end 162.475 79.35) (width 2) (layer B.Cu) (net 18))
 (segment (start 164.3 81.175) (end 164.3 85.15) (width 2) (layer B.Cu) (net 18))
 (segment (start 162.475 79.35) (end 164.3 81.175) (width 2) (layer B.Cu) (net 18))
 (segment (start 162.475 75.655) (end 162.47 75.65) (width 2) (layer B.Cu) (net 18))
 (segment (start 137.2 101.05) (end 137.2 101) (width 0.5) (layer B.Cu) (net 19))
 (segment (start 133.8 101.05) (end 137.2 101.05) (width 0.5) (layer F.Cu) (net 19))
 (via (at 137.2 101.05) (size 2) (drill 0.4) (layers F.Cu B.Cu) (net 19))
 (segment (start 146.4 75.75) (end 148.28 75.75) (width 0.5) (layer B.Cu) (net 19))
 (segment (start 138.9 83.25) (end 146.4 75.75) (width 0.5) (layer B.Cu) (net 19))
 (segment (start 138.9 99.3) (end 138.9 83.25) (width 0.5) (layer B.Cu) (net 19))
 (segment (start 137.2 101) (end 138.9 99.3) (width 0.5) (layer B.Cu) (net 19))
 (segment (start 142.15 85.55) (end 144 85.55) (width 0.5) (layer B.Cu) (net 20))
 (via (at 142.15 85.55) (size 2) (drill 0.4) (layers F.Cu B.Cu) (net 20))
 (segment (start 133.75 85.55) (end 142.15 85.55) (width 0.5) (layer F.Cu) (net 20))
 (segment (start 150.82 78.73) (end 150.82 75.75) (width 0.5) (layer B.Cu) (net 20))
 (segment (start 144 85.55) (end 150.82 78.73) (width 0.5) (layer B.Cu) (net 20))
 (segment (start 148.5796 110.2954) (end 147.55 111.325) (width 0.32) (layer F.Cu) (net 11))
 (segment (start 147.55 111.325) (end 147.525 111.35) (width 0.32) (layer F.Cu) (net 11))
 (segment (start 148.5796 107.394) (end 148.5796 110.2954) (width 0.32) (layer F.Cu) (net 11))
 (segment (start 131.05 81.45) (end 126.15 81.45) (width 0.5) (layer F.Cu) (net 21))
 (segment (start 126.1 81.4) (end 126.1 76.65) (width 0.5) (layer B.Cu) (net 21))
 (segment (start 126.15 81.45) (end 126.1 81.4) (width 0.5) (layer B.Cu) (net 21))
 (via (at 126.15 81.45) (size 2) (drill 0.4) (layers F.Cu B.Cu) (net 21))
 (segment (start 142.1 81.45) (end 142.1 76.6) (width 0.5) (layer F.Cu) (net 22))
 (segment (start 142.05 76.65) (end 138.9 76.65) (width 0.5) (layer B.Cu) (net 22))
 (segment (start 142.1 76.6) (end 142.05 76.65) (width 0.5) (layer B.Cu) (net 22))
 (via (at 142.1 76.6) (size 2) (drill 0.4) (layers F.Cu B.Cu) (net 22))
 (segment (start 149.875 98.1) (end 149.85 98.1) (width 0.5) (layer F.Cu) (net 13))
 (segment (start 144.625 92.875) (end 144.625 89.65) (width 0.5) (layer F.Cu) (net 13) (status 800000))
 (segment (start 149.85 98.1) (end 144.625 92.875) (width 0.5) (layer F.Cu) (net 13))
 (segment (start 149.875 98.05) (end 149.875 98.1) (width 0.32) (layer F.Cu) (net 13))
 (segment (start 149.875 98.1) (end 149.875 102.056) (width 0.32) (layer F.Cu) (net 13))
 (segment (start 147.5 99.275) (end 144.875 99.275) (width 0.5) (layer F.Cu) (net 15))
 (segment (start 141.3 95.7) (end 137.3 95.7) (width 0.5) (layer F.Cu) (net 15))
 (segment (start 144.875 99.275) (end 141.3 95.7) (width 0.5) (layer F.Cu) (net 15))
 (segment (start 137.3 95.7) (end 137.3 90.5) (width 0.5) (layer B.Cu) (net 15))
 (segment (start 137.3 90.5) (end 131.28 84.48) (width 0.5) (layer B.Cu) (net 15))
 (segment (start 131.28 84.48) (end 131.28 76.65) (width 0.5) (layer B.Cu) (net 15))
 (via (at 137.3 95.7) (size 2) (drill 0.4) (layers F.Cu B.Cu) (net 15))
 (segment (start 133.8 95.7) (end 137.3 95.7) (width 0.5) (layer F.Cu) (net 15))
 (segment (start 131.28 76.65) (end 131.28 74.68) (width 0.5) (layer B.Cu) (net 15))
 (segment (start 131.28 74.68) (end 130.25 73.65) (width 0.5) (layer B.Cu) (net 15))
 (segment (start 130.25 73.65) (end 119.75 73.65) (width 0.5) (layer B.Cu) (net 15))
 (segment (start 119.75 73.65) (end 118.48 74.92) (width 0.5) (layer B.Cu) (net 15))
 (segment (start 118.48 74.92) (end 118.48 76.65) (width 0.5) (layer B.Cu) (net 15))
 (segment (start 147.9192 99.6942) (end 147.5 99.275) (width 0.32) (layer F.Cu) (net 15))
 (segment (start 147.5 99.275) (end 147.475 99.25) (width 0.32) (layer F.Cu) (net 15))
 (segment (start 147.9192 102.056) (end 147.9192 99.7058) (width 0.32) (layer F.Cu) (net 15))
 (segment (start 147.9192 99.7058) (end 147.9192 99.6942) (width 0.32) (layer F.Cu) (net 15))
 (segment (start 147.425 98.1) (end 145.175 98.1) (width 0.5) (layer F.Cu) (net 14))
 (segment (start 148.5669 102.056) (end 148.5669 99.2419) (width 0.32) (layer F.Cu) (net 14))
 (segment (start 148.5669 99.2419) (end 147.425 98.1) (width 0.32) (layer F.Cu) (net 14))
 (segment (start 137.575 90.5) (end 133.75 90.5) (width 0.5) (layer F.Cu) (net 14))
 (segment (start 145.175 98.1) (end 137.575 90.5) (width 0.5) (layer F.Cu) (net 14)))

